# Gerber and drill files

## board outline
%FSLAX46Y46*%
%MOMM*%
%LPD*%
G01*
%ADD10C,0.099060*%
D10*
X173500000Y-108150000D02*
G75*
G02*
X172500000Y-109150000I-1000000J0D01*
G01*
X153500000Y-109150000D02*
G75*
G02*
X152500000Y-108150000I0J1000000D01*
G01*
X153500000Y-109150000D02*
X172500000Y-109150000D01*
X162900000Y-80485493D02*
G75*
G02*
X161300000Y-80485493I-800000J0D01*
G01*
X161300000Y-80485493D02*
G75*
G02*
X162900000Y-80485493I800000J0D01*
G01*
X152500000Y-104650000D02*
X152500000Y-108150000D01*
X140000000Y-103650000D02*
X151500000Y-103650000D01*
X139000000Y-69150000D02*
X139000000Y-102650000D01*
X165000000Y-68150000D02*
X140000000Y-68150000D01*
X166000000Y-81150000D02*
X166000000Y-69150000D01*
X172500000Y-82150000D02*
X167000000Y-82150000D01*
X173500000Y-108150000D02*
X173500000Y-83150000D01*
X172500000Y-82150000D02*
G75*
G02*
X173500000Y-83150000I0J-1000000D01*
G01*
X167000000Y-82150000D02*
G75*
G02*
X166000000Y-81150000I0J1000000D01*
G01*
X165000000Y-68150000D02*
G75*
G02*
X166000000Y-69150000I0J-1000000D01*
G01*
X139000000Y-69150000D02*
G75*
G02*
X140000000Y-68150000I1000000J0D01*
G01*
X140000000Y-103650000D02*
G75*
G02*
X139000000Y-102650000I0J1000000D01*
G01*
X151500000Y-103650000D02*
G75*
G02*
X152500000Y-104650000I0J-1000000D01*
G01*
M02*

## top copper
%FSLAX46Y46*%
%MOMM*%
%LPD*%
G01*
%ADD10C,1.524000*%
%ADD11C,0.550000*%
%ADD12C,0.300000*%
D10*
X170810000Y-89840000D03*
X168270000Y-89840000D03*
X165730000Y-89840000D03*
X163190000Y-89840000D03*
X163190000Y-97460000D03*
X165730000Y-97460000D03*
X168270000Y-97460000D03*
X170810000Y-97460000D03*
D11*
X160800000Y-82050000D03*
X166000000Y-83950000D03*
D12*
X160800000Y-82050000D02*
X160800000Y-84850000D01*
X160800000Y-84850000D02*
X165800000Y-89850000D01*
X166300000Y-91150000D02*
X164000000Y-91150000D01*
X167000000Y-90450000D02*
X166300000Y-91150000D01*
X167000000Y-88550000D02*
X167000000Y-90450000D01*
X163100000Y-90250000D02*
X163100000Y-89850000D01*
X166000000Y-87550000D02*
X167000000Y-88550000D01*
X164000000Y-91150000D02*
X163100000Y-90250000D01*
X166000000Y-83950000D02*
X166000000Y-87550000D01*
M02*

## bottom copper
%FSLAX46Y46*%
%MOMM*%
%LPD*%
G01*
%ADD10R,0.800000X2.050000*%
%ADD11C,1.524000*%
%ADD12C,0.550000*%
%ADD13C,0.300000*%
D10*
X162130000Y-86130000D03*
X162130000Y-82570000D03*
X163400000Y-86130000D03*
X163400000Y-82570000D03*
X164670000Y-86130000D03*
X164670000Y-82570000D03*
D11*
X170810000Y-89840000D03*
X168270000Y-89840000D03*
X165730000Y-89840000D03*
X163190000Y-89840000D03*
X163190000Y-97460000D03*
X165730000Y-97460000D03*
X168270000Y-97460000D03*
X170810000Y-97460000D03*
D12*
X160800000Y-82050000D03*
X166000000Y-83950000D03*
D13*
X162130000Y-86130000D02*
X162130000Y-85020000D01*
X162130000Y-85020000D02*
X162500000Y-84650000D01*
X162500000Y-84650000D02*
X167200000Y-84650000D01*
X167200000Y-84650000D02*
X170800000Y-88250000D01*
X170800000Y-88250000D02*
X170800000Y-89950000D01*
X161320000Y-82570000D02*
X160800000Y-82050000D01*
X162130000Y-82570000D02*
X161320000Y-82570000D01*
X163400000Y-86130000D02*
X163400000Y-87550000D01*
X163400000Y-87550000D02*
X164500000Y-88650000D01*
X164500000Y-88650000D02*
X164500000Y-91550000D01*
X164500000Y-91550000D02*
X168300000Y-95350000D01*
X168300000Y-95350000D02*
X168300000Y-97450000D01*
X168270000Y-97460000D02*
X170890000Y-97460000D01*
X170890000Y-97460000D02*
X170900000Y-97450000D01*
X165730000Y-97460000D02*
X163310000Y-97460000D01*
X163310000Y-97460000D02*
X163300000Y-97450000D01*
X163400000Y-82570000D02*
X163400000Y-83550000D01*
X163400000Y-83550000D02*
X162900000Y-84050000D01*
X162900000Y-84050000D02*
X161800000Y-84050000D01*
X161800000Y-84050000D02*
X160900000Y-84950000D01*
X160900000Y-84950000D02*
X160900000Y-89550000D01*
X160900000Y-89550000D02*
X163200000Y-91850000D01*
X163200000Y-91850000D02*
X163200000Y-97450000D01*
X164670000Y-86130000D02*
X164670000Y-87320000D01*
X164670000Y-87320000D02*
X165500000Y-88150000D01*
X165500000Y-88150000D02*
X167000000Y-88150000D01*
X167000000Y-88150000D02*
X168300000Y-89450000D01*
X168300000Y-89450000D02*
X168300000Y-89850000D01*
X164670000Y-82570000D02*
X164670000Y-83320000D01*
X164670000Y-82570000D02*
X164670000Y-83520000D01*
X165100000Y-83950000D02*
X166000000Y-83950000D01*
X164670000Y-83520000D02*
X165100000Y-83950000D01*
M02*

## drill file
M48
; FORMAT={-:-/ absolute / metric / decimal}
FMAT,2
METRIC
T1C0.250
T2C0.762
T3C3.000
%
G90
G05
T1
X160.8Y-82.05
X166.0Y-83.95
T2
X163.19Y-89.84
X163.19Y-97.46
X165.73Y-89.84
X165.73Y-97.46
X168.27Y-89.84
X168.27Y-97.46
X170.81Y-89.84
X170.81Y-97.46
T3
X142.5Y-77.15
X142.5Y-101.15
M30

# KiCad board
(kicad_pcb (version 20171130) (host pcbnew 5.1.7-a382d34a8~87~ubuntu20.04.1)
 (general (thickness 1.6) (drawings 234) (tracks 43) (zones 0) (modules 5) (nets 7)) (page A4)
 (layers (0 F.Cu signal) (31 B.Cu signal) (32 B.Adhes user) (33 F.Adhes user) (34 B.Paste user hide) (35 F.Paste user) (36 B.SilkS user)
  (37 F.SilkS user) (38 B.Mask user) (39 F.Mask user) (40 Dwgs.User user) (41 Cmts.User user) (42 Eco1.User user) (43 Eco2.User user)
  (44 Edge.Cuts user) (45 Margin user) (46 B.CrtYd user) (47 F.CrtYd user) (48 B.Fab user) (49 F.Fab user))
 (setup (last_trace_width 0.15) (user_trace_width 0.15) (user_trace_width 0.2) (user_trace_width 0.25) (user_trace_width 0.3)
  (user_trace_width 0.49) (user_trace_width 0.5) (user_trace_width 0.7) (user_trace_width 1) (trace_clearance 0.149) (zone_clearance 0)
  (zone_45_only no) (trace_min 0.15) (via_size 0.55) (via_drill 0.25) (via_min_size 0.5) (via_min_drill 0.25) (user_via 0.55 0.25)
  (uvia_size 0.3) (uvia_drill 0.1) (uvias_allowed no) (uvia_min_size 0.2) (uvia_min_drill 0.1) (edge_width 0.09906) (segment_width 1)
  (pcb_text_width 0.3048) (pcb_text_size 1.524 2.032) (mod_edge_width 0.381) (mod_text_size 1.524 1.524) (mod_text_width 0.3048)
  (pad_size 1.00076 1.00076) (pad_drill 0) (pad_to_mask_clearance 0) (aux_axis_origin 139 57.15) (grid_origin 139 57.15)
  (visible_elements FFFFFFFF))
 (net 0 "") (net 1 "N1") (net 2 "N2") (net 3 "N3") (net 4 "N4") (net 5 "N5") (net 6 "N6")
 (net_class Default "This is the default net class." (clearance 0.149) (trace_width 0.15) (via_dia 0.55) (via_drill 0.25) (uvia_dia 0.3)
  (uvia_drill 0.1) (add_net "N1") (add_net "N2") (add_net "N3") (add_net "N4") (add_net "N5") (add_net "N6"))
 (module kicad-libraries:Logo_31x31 (layer F.Cu) (at 168.5 104.65)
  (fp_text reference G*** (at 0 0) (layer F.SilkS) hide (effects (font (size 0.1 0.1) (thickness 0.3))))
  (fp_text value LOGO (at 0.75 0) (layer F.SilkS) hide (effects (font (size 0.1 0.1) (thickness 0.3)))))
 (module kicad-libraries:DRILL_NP (layer F.Cu) (at 142.5 101.15)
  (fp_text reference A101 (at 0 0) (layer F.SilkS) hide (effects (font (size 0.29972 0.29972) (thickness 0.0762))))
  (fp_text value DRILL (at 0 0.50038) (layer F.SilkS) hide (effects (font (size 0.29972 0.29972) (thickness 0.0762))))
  (pad "" np_thru_hole circle (at 0 0) (size 2.99974 2.99974) (drill 2.99974) (layers *.Cu *.Mask F.SilkS) (clearance 0.89916)))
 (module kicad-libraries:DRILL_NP (layer F.Cu) (at 142.5 77.15)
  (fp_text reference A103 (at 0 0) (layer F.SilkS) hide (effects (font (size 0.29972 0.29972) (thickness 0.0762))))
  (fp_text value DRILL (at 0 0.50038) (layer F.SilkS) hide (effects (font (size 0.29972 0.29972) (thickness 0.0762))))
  (pad "" np_thru_hole circle (at 0 0) (size 2.99974 2.99974) (drill 2.99974) (layers *.Cu *.Mask F.SilkS) (clearance 0.89916)))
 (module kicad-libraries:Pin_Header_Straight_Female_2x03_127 (layer B.Cu) (at 163.4 84.35)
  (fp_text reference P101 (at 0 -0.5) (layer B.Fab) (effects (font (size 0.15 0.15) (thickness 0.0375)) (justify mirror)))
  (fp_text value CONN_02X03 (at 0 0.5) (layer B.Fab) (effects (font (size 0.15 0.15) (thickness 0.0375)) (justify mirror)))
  (pad 1 smd rect (at -1.27 1.78) (size 0.8 2.05) (layers B.Cu B.Paste B.Mask) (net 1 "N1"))
  (pad 2 smd rect (at -1.27 -1.78) (size 0.8 2.05) (layers B.Cu B.Paste B.Mask) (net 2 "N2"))
  (pad 3 smd rect (at 0 1.78) (size 0.8 2.05) (layers B.Cu B.Paste B.Mask) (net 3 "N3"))
  (pad 4 smd rect (at 0 -1.78) (size 0.8 2.05) (layers B.Cu B.Paste B.Mask) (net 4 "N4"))
  (pad 5 smd rect (at 1.27 1.78) (size 0.8 2.05) (layers B.Cu B.Paste B.Mask) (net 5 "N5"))
  (pad 6 smd rect (at 1.27 -1.78) (size 0.8 2.05) (layers B.Cu B.Paste B.Mask) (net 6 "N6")))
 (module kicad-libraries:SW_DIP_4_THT (layer F.Cu) (at 167 93.65 180)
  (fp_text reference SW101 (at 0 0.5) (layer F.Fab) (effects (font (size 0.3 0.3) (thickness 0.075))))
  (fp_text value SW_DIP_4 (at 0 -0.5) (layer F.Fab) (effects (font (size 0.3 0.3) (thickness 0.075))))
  (pad 1 thru_hole circle (at -3.81 3.81 180) (size 1.524 1.524) (drill 0.762) (layers *.Cu *.Mask F.SilkS) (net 1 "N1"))
  (pad 2 thru_hole circle (at -1.27 3.81 180) (size 1.524 1.524) (drill 0.762) (layers *.Cu *.Mask F.SilkS) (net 5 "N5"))
  (pad 3 thru_hole circle (at 1.27 3.81 180) (size 1.524 1.524) (drill 0.762) (layers *.Cu *.Mask F.SilkS) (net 2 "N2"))
  (pad 4 thru_hole circle (at 3.81 3.81 180) (size 1.524 1.524) (drill 0.762) (layers *.Cu *.Mask F.SilkS) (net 6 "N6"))
  (pad 5 thru_hole circle (at 3.81 -3.81 180) (size 1.524 1.524) (drill 0.762) (layers *.Cu *.Mask F.SilkS) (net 4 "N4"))
  (pad 6 thru_hole circle (at 1.27 -3.81 180) (size 1.524 1.524) (drill 0.762) (layers *.Cu *.Mask F.SilkS) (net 4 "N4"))
  (pad 7 thru_hole circle (at -1.27 -3.81 180) (size 1.524 1.524) (drill 0.762) (layers *.Cu *.Mask F.SilkS) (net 3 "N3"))
  (pad 8 thru_hole circle (at -3.81 -3.81 180) (size 1.524 1.524) (drill 0.762) (layers *.Cu *.Mask F.SilkS) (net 3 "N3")))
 (gr_arc (start 172.5 108.15) (end 172.5 109.15) (angle -90) (layer Edge.Cuts) (width 0.09906))
 (gr_arc (start 153.5 108.15) (end 152.5 108.15) (angle -90) (layer Edge.Cuts) (width 0.09906))
 (gr_line (start 153.5 109.15) (end 172.5 109.15) (layer Edge.Cuts) (width 0.09906))
 (gr_circle (center 162.1 80.485493) (end 162.9 80.485493) (layer Edge.Cuts) (width 0.09906))
 (gr_line (start 152.5 104.65) (end 152.5 108.15) (layer Edge.Cuts) (width 0.09906))
 (gr_line (start 140 103.65) (end 151.5 103.65) (layer Edge.Cuts) (width 0.09906))
 (gr_line (start 139 69.15) (end 139 102.65) (layer Edge.Cuts) (width 0.09906))
 (gr_line (start 165 68.15) (end 140 68.15) (layer Edge.Cuts) (width 0.09906))
 (gr_line (start 166 81.15) (end 166 69.15) (layer Edge.Cuts) (width 0.09906))
 (gr_line (start 172.5 82.15) (end 167 82.15) (layer Edge.Cuts) (width 0.09906))
 (gr_line (start 173.5 108.15) (end 173.5 83.15) (layer Edge.Cuts) (width 0.09906))
 (gr_arc (start 172.5 83.15) (end 173.5 83.15) (angle -90) (layer Edge.Cuts) (width 0.09906))
 (gr_arc (start 167 81.15) (end 166 81.15) (angle -90) (layer Edge.Cuts) (width 0.09906))
 (gr_arc (start 165 69.15) (end 166 69.15) (angle -90) (layer Edge.Cuts) (width 0.09906))
 (gr_arc (start 140 69.15) (end 140 68.15) (angle -90) (layer Edge.Cuts) (width 0.09906))
 (gr_arc (start 140 102.65) (end 139 102.65) (angle -90) (layer Edge.Cuts) (width 0.09906))
 (gr_arc (start 151.5 104.65) (end 152.5 104.65) (angle -90) (layer Edge.Cuts) (width 0.09906))
 (segment (start 162.13 86.13) (end 162.13 85.02) (width 0.3) (layer B.Cu) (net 1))
 (segment (start 162.13 85.02) (end 162.5 84.65) (width 0.3) (layer B.Cu) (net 1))
 (segment (start 162.5 84.65) (end 167.2 84.65) (width 0.3) (layer B.Cu) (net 1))
 (segment (start 167.2 84.65) (end 170.8 88.25) (width 0.3) (layer B.Cu) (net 1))
 (segment (start 170.8 88.25) (end 170.8 89.95) (width 0.3) (layer B.Cu) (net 1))
 (via (at 160.8 82.05) (size 0.55) (drill 0.25) (layers F.Cu B.Cu) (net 2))
 (segment (start 161.32 82.57) (end 160.8 82.05) (width 0.3) (layer B.Cu) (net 2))
 (segment (start 162.13 82.57) (end 161.32 82.57) (width 0.3) (layer B.Cu) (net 2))
 (segment (start 160.8 82.05) (end 160.8 84.85) (width 0.3) (layer F.Cu) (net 2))
 (segment (start 160.8 84.85) (end 165.8 89.85) (width 0.3) (layer F.Cu) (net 2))
 (segment (start 163.4 86.13) (end 163.4 87.55) (width 0.3) (layer B.Cu) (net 3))
 (segment (start 163.4 87.55) (end 164.5 88.65) (width 0.3) (layer B.Cu) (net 3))
 (segment (start 164.5 88.65) (end 164.5 91.55) (width 0.3) (layer B.Cu) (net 3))
 (segment (start 164.5 91.55) (end 168.3 95.35) (width 0.3) (layer B.Cu) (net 3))
 (segment (start 168.3 95.35) (end 168.3 97.45) (width 0.3) (layer B.Cu) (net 3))
 (segment (start 168.27 97.46) (end 170.89 97.46) (width 0.3) (layer B.Cu) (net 3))
 (segment (start 170.89 97.46) (end 170.9 97.45) (width 0.3) (layer B.Cu) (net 3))
 (segment (start 165.73 97.46) (end 163.31 97.46) (width 0.3) (layer B.Cu) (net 4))
 (segment (start 163.31 97.46) (end 163.3 97.45) (width 0.3) (layer B.Cu) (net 4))
 (segment (start 163.4 82.57) (end 163.4 83.55) (width 0.3) (layer B.Cu) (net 4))
 (segment (start 163.4 83.55) (end 162.9 84.05) (width 0.3) (layer B.Cu) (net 4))
 (segment (start 162.9 84.05) (end 161.8 84.05) (width 0.3) (layer B.Cu) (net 4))
 (segment (start 161.8 84.05) (end 160.9 84.95) (width 0.3) (layer B.Cu) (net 4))
 (segment (start 160.9 84.95) (end 160.9 89.55) (width 0.3) (layer B.Cu) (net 4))
 (segment (start 160.9 89.55) (end 163.2 91.85) (width 0.3) (layer B.Cu) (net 4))
 (segment (start 163.2 91.85) (end 163.2 97.45) (width 0.3) (layer B.Cu) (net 4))
 (segment (start 164.67 86.13) (end 164.67 87.32) (width 0.3) (layer B.Cu) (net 5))
 (segment (start 164.67 87.32) (end 165.5 88.15) (width 0.3) (layer B.Cu) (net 5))
 (segment (start 165.5 88.15) (end 167 88.15) (width 0.3) (layer B.Cu) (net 5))
 (segment (start 167 88.15) (end 168.3 89.45) (width 0.3) (layer B.Cu) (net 5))
 (segment (start 168.3 89.45) (end 168.3 89.85) (width 0.3) (layer B.Cu) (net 5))
 (segment (start 164.67 82.57) (end 164.67 83.32) (width 0.3) (layer B.Cu) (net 6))
 (segment (start 164.67 82.57) (end 164.67 83.52) (width 0.3) (layer B.Cu) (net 6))
 (via (at 166 83.95) (size 0.55) (drill 0.25) (layers F.Cu B.Cu) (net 6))
 (segment (start 165.1 83.95) (end 166 83.95) (width 0.3) (layer B.Cu) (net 6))
 (segment (start 164.67 83.52) (end 165.1 83.95) (width 0.3) (layer B.Cu) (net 6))
 (segment (start 166.3 91.15) (end 164 91.15) (width 0.3) (layer F.Cu) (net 6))
 (segment (start 167 90.45) (end 166.3 91.15) (width 0.3) (layer F.Cu) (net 6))
 (segment (start 167 88.55) (end 167 90.45) (width 0.3) (layer F.Cu) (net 6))
 (segment (start 163.1 90.25) (end 163.1 89.85) (width 0.3) (layer F.Cu) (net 6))
 (segment (start 166 87.55) (end 167 88.55) (width 0.3) (layer F.Cu) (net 6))
 (segment (start 164 91.15) (end 163.1 90.25) (width 0.3) (layer F.Cu) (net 6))
 (segment (start 166 83.95) (end 166 87.55) (width 0.3) (layer F.Cu) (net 6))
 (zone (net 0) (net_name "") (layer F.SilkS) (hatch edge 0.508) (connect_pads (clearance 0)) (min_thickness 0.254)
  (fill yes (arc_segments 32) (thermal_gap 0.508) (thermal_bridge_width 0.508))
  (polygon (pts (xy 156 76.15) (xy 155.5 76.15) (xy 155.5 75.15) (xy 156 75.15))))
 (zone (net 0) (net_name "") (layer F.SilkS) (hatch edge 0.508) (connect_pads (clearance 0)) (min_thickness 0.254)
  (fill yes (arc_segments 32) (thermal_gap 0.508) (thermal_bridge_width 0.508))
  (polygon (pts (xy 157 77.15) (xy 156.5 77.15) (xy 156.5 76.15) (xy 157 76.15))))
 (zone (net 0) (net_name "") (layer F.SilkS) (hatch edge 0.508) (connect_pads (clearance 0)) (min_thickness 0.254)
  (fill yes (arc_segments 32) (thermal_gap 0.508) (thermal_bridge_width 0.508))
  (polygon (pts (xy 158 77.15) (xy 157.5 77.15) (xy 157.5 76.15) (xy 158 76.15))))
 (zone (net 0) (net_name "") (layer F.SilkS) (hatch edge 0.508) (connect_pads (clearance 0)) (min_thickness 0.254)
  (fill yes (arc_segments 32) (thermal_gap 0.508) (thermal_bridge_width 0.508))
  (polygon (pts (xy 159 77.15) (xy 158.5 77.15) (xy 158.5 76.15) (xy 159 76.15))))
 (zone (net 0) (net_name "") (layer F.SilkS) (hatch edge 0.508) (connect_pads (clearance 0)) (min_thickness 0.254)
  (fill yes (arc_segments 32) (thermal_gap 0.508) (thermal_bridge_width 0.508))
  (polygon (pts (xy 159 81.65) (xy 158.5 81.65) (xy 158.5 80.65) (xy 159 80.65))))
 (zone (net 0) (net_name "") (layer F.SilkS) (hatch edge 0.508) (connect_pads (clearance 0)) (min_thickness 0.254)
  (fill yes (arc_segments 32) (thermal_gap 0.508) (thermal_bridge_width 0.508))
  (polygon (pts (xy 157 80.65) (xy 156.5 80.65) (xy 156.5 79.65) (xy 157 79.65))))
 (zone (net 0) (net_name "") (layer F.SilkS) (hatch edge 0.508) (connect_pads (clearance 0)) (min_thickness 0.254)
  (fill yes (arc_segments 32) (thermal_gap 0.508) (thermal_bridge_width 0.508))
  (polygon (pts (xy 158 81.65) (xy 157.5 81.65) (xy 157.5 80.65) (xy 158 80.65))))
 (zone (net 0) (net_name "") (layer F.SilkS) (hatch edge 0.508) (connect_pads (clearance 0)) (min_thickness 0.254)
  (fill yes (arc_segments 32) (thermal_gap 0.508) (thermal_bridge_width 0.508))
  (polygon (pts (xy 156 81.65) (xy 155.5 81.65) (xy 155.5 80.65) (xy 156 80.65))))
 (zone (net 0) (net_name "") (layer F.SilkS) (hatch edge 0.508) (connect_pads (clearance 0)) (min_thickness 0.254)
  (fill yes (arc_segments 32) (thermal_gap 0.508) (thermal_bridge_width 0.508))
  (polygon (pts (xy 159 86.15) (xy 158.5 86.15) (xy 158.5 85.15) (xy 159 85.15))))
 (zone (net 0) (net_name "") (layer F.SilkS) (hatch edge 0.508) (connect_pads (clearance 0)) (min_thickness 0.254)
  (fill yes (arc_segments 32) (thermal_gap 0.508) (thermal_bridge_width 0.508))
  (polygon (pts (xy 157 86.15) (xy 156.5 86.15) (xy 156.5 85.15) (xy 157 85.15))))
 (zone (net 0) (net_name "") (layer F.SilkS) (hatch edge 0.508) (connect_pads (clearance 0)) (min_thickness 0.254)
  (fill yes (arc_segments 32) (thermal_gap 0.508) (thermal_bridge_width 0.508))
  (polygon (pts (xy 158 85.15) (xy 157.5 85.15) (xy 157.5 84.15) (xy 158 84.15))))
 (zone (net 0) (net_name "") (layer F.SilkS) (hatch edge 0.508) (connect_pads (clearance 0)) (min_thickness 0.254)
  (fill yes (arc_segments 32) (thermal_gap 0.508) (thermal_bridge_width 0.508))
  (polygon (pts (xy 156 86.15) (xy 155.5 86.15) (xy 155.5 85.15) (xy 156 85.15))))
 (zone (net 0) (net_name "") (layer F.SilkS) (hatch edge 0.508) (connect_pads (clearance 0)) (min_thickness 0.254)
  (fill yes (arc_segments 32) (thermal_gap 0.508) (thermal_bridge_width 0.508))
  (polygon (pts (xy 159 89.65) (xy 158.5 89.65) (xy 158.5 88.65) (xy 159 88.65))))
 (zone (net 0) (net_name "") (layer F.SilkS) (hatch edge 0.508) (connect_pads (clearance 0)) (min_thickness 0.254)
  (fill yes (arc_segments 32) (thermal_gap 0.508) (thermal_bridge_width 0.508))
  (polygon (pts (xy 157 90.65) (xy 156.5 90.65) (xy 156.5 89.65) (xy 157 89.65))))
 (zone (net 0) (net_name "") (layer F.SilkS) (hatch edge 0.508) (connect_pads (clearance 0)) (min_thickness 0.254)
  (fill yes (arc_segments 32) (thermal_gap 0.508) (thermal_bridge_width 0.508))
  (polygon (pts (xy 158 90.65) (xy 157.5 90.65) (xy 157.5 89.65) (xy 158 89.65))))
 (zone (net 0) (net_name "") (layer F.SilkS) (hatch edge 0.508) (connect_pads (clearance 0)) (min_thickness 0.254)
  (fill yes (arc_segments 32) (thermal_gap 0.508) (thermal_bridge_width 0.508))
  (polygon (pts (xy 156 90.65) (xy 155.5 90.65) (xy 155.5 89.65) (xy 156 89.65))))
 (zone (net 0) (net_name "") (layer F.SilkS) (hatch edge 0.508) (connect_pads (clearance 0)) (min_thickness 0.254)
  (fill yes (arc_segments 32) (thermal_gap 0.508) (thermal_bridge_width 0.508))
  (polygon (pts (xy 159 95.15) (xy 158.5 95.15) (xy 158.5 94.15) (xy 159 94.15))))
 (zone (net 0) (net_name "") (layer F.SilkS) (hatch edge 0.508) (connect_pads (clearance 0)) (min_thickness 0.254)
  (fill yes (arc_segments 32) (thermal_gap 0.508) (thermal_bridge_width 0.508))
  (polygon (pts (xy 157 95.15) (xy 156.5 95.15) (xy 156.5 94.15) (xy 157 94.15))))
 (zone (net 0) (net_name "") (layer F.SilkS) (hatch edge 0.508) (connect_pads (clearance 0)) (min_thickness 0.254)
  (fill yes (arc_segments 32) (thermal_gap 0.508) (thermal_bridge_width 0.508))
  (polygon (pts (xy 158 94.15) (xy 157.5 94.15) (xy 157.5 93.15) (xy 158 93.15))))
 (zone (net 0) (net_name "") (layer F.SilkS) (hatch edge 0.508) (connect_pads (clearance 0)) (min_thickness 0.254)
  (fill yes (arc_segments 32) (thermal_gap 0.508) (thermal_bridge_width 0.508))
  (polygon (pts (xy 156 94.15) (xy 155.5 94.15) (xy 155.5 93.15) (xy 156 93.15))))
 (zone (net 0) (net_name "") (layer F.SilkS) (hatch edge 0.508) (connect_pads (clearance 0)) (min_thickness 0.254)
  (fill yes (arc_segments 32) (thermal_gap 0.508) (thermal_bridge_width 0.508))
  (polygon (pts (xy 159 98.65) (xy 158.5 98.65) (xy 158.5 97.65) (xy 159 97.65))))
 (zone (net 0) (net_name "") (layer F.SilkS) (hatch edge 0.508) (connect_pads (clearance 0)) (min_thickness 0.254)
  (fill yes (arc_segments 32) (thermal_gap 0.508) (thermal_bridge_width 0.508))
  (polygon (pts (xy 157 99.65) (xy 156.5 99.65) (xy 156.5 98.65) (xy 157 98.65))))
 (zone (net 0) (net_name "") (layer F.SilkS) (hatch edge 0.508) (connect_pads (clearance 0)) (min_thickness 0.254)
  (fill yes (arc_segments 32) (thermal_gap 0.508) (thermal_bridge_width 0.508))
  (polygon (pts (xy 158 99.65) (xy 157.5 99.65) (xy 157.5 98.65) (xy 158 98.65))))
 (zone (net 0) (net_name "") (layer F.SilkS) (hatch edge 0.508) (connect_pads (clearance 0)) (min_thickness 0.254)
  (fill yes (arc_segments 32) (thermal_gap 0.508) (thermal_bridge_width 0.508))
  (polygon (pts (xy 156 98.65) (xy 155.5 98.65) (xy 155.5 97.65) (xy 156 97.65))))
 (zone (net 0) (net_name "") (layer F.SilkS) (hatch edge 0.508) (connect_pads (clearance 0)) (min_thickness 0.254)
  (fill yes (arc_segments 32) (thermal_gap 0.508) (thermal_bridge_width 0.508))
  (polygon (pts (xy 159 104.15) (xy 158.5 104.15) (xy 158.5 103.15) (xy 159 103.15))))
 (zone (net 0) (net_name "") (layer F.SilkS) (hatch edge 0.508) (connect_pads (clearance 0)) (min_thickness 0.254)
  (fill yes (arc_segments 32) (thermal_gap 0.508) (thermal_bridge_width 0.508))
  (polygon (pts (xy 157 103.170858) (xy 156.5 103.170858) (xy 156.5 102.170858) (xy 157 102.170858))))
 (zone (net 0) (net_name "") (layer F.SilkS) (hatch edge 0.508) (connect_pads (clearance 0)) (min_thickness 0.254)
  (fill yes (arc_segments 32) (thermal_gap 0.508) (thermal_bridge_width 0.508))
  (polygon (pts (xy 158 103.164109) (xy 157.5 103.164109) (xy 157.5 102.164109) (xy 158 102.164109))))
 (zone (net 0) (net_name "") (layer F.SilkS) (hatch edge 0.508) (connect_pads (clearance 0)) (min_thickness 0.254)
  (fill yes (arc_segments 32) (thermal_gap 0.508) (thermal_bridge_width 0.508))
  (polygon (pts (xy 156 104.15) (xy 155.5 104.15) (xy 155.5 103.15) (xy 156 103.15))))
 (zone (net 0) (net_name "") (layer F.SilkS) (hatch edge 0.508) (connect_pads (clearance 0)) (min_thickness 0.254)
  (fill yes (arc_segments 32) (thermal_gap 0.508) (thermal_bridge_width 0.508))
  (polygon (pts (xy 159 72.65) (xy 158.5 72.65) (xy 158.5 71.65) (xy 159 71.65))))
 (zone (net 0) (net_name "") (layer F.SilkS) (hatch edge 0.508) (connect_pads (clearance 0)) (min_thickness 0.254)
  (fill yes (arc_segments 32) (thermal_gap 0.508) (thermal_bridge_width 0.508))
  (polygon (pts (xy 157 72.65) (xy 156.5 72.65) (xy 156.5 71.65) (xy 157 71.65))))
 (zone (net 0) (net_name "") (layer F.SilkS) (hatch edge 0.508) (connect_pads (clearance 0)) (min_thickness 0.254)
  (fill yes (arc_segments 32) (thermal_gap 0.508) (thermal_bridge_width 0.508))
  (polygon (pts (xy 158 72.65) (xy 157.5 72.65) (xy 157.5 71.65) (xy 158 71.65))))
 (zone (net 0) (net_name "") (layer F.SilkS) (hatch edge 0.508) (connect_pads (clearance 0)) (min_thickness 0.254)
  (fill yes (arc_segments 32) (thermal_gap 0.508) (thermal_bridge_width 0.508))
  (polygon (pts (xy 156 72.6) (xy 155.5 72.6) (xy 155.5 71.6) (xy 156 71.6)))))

